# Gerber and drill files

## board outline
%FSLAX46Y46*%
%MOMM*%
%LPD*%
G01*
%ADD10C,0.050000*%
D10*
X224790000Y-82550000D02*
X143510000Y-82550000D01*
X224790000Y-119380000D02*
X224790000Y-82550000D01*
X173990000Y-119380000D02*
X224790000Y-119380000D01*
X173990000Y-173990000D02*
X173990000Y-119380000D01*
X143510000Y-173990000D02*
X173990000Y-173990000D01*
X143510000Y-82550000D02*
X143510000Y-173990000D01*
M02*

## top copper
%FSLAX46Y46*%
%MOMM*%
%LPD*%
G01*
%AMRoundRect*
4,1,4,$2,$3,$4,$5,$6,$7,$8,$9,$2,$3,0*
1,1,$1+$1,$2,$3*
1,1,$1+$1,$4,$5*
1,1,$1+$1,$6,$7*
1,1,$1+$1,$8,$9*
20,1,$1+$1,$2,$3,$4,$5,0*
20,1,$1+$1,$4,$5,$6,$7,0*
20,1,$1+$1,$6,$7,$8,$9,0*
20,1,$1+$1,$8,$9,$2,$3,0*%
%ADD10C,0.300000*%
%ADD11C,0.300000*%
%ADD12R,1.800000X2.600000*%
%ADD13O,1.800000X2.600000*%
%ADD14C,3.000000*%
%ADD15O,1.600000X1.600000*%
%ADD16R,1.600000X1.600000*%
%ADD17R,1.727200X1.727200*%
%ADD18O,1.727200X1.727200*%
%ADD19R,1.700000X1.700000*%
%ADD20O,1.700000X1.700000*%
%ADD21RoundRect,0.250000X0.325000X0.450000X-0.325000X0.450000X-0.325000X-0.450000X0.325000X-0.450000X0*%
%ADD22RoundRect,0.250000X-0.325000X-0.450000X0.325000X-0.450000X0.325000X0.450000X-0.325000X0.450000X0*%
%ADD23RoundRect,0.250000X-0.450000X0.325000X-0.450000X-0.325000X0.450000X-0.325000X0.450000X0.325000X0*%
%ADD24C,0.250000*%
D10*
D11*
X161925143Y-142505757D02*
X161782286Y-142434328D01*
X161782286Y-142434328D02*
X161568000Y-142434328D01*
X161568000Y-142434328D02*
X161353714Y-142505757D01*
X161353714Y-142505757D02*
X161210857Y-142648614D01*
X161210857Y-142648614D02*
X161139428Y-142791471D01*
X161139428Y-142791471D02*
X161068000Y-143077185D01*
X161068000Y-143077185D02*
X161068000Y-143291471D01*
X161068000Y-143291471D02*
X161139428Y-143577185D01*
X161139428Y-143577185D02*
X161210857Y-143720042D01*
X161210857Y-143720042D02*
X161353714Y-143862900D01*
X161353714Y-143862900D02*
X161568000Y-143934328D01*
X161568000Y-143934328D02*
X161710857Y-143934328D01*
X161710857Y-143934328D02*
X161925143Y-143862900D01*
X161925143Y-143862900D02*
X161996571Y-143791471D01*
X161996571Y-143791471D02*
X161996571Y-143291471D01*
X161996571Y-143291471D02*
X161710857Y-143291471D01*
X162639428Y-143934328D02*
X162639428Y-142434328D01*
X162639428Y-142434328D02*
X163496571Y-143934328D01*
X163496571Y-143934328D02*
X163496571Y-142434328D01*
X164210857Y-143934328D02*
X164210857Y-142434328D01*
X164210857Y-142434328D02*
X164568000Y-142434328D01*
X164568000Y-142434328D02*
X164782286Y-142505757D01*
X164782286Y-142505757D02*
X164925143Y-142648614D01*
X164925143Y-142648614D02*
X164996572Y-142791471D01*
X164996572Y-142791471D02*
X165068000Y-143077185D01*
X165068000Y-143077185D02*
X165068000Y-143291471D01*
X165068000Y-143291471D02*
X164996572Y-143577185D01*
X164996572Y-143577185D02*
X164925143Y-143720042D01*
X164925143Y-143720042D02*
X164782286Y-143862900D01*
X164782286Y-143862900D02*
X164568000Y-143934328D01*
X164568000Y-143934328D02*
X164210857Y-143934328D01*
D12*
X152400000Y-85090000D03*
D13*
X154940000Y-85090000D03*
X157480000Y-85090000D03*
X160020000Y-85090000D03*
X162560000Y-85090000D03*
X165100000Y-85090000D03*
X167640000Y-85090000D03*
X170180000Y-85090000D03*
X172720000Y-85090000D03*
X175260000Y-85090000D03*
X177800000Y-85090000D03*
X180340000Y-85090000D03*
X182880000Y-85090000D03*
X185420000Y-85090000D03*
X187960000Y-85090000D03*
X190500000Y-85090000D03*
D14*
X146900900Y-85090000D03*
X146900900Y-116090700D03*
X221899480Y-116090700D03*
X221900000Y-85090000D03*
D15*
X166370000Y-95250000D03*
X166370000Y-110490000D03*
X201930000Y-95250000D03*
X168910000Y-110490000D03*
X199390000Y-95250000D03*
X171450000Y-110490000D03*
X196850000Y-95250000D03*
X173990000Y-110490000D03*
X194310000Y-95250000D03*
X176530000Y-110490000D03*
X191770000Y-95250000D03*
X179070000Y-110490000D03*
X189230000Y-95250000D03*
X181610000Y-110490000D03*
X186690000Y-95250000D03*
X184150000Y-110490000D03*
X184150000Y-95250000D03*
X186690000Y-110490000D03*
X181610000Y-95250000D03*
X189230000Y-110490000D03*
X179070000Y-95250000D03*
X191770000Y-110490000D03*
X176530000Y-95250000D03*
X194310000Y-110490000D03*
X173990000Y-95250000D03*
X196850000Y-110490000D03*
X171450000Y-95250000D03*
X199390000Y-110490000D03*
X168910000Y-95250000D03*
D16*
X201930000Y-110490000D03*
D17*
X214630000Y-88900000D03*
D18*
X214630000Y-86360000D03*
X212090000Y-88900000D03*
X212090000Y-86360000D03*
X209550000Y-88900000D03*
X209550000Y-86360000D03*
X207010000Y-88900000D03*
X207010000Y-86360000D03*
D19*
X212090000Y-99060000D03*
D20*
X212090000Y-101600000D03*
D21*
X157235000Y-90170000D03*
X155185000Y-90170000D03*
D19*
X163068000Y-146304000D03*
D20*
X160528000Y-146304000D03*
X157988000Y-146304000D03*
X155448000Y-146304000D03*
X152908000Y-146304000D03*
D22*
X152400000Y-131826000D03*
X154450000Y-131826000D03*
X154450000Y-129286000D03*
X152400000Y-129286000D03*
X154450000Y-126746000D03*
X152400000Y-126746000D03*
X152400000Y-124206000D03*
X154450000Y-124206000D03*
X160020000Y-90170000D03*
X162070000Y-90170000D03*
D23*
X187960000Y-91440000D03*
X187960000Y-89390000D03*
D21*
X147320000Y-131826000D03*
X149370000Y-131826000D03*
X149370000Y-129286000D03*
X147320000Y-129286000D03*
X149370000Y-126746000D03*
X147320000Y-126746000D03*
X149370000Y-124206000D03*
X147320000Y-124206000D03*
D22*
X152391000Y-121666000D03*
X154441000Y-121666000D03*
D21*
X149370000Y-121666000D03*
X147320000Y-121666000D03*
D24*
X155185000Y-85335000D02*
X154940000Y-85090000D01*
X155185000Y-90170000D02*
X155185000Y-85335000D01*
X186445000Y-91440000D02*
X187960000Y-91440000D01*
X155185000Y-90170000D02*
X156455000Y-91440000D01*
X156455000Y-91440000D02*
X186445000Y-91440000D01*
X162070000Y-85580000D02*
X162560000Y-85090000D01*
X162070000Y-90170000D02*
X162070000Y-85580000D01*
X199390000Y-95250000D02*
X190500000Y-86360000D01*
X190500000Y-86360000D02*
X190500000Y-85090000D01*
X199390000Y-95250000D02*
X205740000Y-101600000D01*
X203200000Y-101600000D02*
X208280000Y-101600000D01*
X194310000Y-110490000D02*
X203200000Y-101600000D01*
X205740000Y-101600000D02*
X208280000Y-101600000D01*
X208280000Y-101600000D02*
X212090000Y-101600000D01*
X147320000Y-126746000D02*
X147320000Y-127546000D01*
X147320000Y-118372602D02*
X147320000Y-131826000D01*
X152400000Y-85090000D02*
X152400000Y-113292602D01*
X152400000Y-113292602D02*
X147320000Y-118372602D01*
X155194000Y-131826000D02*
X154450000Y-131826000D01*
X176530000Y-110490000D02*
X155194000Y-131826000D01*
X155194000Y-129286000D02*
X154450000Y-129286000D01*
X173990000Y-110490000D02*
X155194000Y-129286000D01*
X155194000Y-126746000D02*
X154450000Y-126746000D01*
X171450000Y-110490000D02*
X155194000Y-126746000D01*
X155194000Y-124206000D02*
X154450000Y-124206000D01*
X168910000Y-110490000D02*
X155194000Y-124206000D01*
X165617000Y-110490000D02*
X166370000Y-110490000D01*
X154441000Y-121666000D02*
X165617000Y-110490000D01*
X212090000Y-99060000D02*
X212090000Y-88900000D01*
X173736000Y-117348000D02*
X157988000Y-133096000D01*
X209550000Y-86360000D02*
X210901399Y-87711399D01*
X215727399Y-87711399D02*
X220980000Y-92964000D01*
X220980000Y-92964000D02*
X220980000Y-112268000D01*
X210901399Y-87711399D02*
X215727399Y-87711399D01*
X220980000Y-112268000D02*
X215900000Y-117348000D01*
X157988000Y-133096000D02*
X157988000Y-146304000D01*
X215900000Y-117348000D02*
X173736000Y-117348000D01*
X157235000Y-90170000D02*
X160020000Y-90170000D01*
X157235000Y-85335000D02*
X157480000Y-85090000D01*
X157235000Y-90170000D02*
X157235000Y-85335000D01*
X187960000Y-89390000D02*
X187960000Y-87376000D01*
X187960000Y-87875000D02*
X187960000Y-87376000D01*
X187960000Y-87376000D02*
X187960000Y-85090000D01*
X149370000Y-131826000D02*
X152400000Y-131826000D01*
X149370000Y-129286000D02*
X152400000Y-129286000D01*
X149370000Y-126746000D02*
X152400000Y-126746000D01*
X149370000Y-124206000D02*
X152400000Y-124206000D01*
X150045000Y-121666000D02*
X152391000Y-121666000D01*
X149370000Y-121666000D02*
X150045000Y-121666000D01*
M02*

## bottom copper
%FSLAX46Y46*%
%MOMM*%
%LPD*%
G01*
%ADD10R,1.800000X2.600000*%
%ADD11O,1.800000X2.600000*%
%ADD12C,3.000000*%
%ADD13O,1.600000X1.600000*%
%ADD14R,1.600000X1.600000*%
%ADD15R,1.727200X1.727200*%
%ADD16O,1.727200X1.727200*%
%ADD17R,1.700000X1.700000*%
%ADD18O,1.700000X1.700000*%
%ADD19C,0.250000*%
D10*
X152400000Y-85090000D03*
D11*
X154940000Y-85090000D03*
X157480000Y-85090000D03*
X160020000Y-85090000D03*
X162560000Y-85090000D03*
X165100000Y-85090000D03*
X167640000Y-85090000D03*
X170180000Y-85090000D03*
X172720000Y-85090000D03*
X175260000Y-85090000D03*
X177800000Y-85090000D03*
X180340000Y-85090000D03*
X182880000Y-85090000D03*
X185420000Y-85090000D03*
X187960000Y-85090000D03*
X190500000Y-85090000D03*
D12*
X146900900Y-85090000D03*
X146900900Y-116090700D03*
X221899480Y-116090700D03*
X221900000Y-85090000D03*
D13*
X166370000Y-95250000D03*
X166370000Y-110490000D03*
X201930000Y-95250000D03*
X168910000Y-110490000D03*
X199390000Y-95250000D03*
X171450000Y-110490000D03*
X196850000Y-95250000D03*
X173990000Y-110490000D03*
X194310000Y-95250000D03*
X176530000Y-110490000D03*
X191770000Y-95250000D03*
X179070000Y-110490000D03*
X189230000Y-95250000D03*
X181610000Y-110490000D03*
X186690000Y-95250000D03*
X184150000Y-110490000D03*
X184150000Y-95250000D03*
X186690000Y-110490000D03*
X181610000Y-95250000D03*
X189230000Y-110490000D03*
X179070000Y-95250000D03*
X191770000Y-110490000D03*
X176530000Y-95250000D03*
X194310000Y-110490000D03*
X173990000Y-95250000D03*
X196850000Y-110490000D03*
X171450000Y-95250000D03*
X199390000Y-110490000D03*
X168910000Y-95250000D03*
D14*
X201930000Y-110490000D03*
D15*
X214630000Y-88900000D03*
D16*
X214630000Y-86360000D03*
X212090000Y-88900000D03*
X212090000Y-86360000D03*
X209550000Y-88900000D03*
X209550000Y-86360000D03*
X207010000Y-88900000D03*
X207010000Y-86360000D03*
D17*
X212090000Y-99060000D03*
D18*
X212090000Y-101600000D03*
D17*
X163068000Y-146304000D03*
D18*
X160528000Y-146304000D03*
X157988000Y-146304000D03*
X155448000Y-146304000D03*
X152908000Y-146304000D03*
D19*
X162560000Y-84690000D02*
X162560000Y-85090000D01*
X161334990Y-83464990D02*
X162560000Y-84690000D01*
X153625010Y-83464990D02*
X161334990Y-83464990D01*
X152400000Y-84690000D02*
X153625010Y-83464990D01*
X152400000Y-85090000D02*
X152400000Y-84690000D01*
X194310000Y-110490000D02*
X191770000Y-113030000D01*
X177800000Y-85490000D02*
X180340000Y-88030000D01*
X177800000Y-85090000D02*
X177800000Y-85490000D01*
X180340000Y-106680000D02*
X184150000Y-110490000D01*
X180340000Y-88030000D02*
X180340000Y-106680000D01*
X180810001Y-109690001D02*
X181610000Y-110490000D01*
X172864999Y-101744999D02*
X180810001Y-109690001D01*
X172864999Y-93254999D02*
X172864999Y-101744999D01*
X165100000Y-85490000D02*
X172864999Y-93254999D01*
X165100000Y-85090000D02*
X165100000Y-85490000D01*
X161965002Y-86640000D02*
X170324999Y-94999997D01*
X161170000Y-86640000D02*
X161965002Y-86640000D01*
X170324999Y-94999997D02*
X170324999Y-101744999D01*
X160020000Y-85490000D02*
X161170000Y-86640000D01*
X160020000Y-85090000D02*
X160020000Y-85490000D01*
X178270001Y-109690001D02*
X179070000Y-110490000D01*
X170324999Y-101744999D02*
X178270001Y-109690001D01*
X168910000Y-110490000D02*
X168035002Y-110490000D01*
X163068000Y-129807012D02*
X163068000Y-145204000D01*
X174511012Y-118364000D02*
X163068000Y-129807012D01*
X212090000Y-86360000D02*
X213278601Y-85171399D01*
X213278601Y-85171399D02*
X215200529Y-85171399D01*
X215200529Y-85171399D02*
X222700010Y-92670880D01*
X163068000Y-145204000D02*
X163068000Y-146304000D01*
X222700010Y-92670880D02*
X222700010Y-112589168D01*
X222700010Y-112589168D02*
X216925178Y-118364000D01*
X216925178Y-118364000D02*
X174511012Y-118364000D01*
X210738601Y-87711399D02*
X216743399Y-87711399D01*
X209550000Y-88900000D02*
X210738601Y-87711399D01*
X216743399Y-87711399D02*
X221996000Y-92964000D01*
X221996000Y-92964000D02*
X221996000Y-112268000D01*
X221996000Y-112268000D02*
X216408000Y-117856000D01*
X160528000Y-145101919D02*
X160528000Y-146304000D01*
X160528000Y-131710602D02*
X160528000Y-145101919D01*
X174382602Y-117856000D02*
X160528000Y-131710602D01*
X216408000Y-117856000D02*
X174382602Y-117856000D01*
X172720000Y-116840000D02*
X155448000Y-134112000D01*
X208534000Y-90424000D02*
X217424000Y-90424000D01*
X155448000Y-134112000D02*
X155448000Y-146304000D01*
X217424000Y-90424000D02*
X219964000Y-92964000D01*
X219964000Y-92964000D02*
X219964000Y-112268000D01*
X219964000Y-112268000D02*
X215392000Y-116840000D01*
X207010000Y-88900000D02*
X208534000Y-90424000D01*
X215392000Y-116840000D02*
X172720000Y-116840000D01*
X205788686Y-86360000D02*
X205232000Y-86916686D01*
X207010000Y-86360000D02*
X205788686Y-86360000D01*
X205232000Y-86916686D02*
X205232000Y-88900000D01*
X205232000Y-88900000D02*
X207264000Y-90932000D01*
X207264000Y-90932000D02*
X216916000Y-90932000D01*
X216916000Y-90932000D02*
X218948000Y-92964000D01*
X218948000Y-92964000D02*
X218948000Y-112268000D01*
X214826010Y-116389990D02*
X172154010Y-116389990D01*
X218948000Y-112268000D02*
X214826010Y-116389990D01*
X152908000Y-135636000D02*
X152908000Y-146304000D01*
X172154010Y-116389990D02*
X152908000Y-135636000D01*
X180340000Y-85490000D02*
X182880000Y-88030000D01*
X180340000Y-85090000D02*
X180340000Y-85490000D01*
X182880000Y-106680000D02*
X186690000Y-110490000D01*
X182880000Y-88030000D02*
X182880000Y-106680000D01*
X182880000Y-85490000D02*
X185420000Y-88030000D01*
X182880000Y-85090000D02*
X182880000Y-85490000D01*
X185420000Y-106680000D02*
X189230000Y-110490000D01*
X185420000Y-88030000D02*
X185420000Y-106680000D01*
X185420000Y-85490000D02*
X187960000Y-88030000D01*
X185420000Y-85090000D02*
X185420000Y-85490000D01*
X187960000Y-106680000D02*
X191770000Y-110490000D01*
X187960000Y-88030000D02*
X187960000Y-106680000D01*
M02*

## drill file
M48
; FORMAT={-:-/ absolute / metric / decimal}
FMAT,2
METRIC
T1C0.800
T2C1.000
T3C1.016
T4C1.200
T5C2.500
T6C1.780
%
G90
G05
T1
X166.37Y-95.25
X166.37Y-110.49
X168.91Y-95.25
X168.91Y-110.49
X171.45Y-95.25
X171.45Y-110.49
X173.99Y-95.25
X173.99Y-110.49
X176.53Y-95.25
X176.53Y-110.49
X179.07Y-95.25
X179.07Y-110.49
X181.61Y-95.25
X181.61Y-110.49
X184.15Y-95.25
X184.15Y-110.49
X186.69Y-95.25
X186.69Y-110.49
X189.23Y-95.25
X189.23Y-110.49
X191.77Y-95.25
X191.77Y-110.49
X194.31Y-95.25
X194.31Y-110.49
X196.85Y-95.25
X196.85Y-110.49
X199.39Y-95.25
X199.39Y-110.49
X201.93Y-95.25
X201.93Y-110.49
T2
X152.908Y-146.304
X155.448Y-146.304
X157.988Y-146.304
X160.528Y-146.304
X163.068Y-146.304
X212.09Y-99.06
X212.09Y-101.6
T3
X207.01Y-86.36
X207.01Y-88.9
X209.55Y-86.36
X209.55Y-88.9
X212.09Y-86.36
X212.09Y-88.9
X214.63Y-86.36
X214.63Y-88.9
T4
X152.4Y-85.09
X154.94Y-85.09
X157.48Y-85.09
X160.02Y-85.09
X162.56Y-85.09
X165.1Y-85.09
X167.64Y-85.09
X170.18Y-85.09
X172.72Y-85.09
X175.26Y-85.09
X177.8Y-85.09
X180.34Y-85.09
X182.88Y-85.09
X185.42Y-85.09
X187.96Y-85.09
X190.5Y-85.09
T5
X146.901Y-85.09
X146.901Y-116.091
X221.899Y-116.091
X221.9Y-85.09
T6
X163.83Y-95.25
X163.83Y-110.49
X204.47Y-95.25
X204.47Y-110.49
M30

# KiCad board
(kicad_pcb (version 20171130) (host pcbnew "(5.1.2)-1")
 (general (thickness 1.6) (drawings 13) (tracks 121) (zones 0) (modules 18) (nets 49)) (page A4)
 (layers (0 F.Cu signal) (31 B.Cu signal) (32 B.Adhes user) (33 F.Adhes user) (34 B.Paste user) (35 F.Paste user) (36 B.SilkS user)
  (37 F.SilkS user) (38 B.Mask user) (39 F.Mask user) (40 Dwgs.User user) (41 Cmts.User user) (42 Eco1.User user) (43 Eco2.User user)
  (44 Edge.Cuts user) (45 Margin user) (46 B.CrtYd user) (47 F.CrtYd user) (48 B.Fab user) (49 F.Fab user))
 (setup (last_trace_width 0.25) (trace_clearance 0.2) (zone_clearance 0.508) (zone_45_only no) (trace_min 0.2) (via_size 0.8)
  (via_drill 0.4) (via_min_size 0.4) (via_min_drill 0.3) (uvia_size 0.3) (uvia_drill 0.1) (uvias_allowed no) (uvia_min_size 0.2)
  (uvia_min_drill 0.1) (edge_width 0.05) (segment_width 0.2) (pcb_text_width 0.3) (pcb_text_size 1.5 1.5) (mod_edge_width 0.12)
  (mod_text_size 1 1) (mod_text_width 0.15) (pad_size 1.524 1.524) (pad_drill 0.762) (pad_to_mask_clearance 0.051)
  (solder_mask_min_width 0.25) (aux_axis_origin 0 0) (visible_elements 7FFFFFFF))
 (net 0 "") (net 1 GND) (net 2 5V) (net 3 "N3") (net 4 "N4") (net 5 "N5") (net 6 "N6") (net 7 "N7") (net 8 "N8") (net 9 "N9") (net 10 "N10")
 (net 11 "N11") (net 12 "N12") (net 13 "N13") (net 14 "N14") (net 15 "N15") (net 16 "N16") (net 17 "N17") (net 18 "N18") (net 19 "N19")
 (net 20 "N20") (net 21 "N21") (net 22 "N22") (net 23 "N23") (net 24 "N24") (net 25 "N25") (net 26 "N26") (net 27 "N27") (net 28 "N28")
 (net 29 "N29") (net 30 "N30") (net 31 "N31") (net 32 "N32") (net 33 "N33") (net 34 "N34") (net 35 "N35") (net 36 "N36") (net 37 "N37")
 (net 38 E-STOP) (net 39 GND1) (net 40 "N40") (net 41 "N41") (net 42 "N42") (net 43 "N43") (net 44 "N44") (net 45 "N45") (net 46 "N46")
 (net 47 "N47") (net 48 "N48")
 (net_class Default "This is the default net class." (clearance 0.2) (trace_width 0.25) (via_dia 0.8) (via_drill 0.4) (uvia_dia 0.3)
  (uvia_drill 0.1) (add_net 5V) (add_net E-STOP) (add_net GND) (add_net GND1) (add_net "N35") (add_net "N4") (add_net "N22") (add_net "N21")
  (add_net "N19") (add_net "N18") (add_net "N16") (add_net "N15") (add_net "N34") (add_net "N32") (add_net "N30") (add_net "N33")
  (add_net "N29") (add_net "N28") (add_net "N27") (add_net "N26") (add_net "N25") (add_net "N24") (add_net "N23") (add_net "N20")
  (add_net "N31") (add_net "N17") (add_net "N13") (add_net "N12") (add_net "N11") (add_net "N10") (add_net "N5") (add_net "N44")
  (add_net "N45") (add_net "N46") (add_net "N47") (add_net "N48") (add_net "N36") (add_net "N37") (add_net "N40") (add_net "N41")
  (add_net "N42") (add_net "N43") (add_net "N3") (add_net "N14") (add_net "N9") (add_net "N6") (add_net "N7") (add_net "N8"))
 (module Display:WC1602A (layer F.Cu) (at 152.4 85.09)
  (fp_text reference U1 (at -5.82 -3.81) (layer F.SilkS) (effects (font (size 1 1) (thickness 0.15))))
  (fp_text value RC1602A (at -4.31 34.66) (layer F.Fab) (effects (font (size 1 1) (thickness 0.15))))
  (pad 1 thru_hole rect (at 0 0) (size 1.8 2.6) (drill 1.2) (layers *.Cu *.Mask) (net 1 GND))
  (pad 2 thru_hole oval (at 2.54 0) (size 1.8 2.6) (drill 1.2) (layers *.Cu *.Mask) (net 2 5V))
  (pad 3 thru_hole oval (at 5.08 0) (size 1.8 2.6) (drill 1.2) (layers *.Cu *.Mask) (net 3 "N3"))
  (pad 4 thru_hole oval (at 7.62 0) (size 1.8 2.6) (drill 1.2) (layers *.Cu *.Mask) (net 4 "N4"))
  (pad 5 thru_hole oval (at 10.16 0) (size 1.8 2.6) (drill 1.2) (layers *.Cu *.Mask) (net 1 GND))
  (pad 6 thru_hole oval (at 12.7 0) (size 1.8 2.6) (drill 1.2) (layers *.Cu *.Mask) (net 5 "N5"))
  (pad 7 thru_hole oval (at 15.24 0) (size 1.8 2.6) (drill 1.2) (layers *.Cu *.Mask) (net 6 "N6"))
  (pad 8 thru_hole oval (at 17.78 0) (size 1.8 2.6) (drill 1.2) (layers *.Cu *.Mask) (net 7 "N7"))
  (pad 9 thru_hole oval (at 20.32 0) (size 1.8 2.6) (drill 1.2) (layers *.Cu *.Mask) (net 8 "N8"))
  (pad 10 thru_hole oval (at 22.86 0) (size 1.8 2.6) (drill 1.2) (layers *.Cu *.Mask) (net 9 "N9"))
  (pad 11 thru_hole oval (at 25.4 0) (size 1.8 2.6) (drill 1.2) (layers *.Cu *.Mask) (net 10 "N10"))
  (pad 12 thru_hole oval (at 27.94 0) (size 1.8 2.6) (drill 1.2) (layers *.Cu *.Mask) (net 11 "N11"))
  (pad 13 thru_hole oval (at 30.48 0) (size 1.8 2.6) (drill 1.2) (layers *.Cu *.Mask) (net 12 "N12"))
  (pad 14 thru_hole oval (at 33.02 0) (size 1.8 2.6) (drill 1.2) (layers *.Cu *.Mask) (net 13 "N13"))
  (pad 15 thru_hole oval (at 35.56 0) (size 1.8 2.6) (drill 1.2) (layers *.Cu *.Mask) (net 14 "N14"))
  (pad 16 thru_hole oval (at 38.1 0) (size 1.8 2.6) (drill 1.2) (layers *.Cu *.Mask) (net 1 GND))
  (pad "" thru_hole circle (at -5.4991 0) (size 3 3) (drill 2.5) (layers *.Cu *.Mask))
  (pad "" thru_hole circle (at -5.4991 31.0007) (size 3 3) (drill 2.5) (layers *.Cu *.Mask))
  (pad "" thru_hole circle (at 69.49948 31.0007) (size 3 3) (drill 2.5) (layers *.Cu *.Mask))
  (pad "" thru_hole circle (at 69.5 0) (size 3 3) (drill 2.5) (layers *.Cu *.Mask)))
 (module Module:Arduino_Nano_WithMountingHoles (layer B.Cu) (at 201.93 110.49 90)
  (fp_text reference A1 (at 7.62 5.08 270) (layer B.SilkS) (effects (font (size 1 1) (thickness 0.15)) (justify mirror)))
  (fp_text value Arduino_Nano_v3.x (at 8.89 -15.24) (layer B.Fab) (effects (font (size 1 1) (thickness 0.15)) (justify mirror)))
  (pad "" np_thru_hole circle (at 0 -38.1 90) (size 1.78 1.78) (drill 1.78) (layers *.Cu *.Mask))
  (pad "" np_thru_hole circle (at 15.24 -38.1 90) (size 1.78 1.78) (drill 1.78) (layers *.Cu *.Mask))
  (pad "" np_thru_hole circle (at 15.24 2.54 90) (size 1.78 1.78) (drill 1.78) (layers *.Cu *.Mask))
  (pad "" np_thru_hole circle (at 0 2.54 90) (size 1.78 1.78) (drill 1.78) (layers *.Cu *.Mask))
  (pad 16 thru_hole oval (at 15.24 -35.56 90) (size 1.6 1.6) (drill 0.8) (layers *.Cu *.Mask) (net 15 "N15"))
  (pad 15 thru_hole oval (at 0 -35.56 90) (size 1.6 1.6) (drill 0.8) (layers *.Cu *.Mask) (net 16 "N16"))
  (pad 30 thru_hole oval (at 15.24 0 90) (size 1.6 1.6) (drill 0.8) (layers *.Cu *.Mask) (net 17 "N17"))
  (pad 14 thru_hole oval (at 0 -33.02 90) (size 1.6 1.6) (drill 0.8) (layers *.Cu *.Mask) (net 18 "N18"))
  (pad 29 thru_hole oval (at 15.24 -2.54 90) (size 1.6 1.6) (drill 0.8) (layers *.Cu *.Mask) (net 1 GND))
  (pad 13 thru_hole oval (at 0 -30.48 90) (size 1.6 1.6) (drill 0.8) (layers *.Cu *.Mask) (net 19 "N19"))
  (pad 28 thru_hole oval (at 15.24 -5.08 90) (size 1.6 1.6) (drill 0.8) (layers *.Cu *.Mask) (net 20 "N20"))
  (pad 12 thru_hole oval (at 0 -27.94 90) (size 1.6 1.6) (drill 0.8) (layers *.Cu *.Mask) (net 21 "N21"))
  (pad 27 thru_hole oval (at 15.24 -7.62 90) (size 1.6 1.6) (drill 0.8) (layers *.Cu *.Mask) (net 2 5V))
  (pad 11 thru_hole oval (at 0 -25.4 90) (size 1.6 1.6) (drill 0.8) (layers *.Cu *.Mask) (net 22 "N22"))
  (pad 26 thru_hole oval (at 15.24 -10.16 90) (size 1.6 1.6) (drill 0.8) (layers *.Cu *.Mask) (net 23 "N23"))
  (pad 10 thru_hole oval (at 0 -22.86 90) (size 1.6 1.6) (drill 0.8) (layers *.Cu *.Mask) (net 4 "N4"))
  (pad 25 thru_hole oval (at 15.24 -12.7 90) (size 1.6 1.6) (drill 0.8) (layers *.Cu *.Mask) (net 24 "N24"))
  (pad 9 thru_hole oval (at 0 -20.32 90) (size 1.6 1.6) (drill 0.8) (layers *.Cu *.Mask) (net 5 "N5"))
  (pad 24 thru_hole oval (at 15.24 -15.24 90) (size 1.6 1.6) (drill 0.8) (layers *.Cu *.Mask) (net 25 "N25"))
  (pad 8 thru_hole oval (at 0 -17.78 90) (size 1.6 1.6) (drill 0.8) (layers *.Cu *.Mask) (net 10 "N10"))
  (pad 23 thru_hole oval (at 15.24 -17.78 90) (size 1.6 1.6) (drill 0.8) (layers *.Cu *.Mask) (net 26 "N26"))
  (pad 7 thru_hole oval (at 0 -15.24 90) (size 1.6 1.6) (drill 0.8) (layers *.Cu *.Mask) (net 11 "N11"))
  (pad 22 thru_hole oval (at 15.24 -20.32 90) (size 1.6 1.6) (drill 0.8) (layers *.Cu *.Mask) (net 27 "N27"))
  (pad 6 thru_hole oval (at 0 -12.7 90) (size 1.6 1.6) (drill 0.8) (layers *.Cu *.Mask) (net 12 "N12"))
  (pad 21 thru_hole oval (at 15.24 -22.86 90) (size 1.6 1.6) (drill 0.8) (layers *.Cu *.Mask) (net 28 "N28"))
  (pad 5 thru_hole oval (at 0 -10.16 90) (size 1.6 1.6) (drill 0.8) (layers *.Cu *.Mask) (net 13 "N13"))
  (pad 20 thru_hole oval (at 15.24 -25.4 90) (size 1.6 1.6) (drill 0.8) (layers *.Cu *.Mask) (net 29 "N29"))
  (pad 4 thru_hole oval (at 0 -7.62 90) (size 1.6 1.6) (drill 0.8) (layers *.Cu *.Mask) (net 1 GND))
  (pad 19 thru_hole oval (at 15.24 -27.94 90) (size 1.6 1.6) (drill 0.8) (layers *.Cu *.Mask) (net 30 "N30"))
  (pad 3 thru_hole oval (at 0 -5.08 90) (size 1.6 1.6) (drill 0.8) (layers *.Cu *.Mask) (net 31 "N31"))
  (pad 18 thru_hole oval (at 15.24 -30.48 90) (size 1.6 1.6) (drill 0.8) (layers *.Cu *.Mask) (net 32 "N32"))
  (pad 2 thru_hole oval (at 0 -2.54 90) (size 1.6 1.6) (drill 0.8) (layers *.Cu *.Mask) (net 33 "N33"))
  (pad 17 thru_hole oval (at 15.24 -33.02 90) (size 1.6 1.6) (drill 0.8) (layers *.Cu *.Mask) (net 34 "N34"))
  (pad 1 thru_hole rect (at 0 0 90) (size 1.6 1.6) (drill 0.8) (layers *.Cu *.Mask) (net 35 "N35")))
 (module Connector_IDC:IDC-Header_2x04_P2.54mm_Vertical (layer B.Cu) (at 214.63 88.9 90)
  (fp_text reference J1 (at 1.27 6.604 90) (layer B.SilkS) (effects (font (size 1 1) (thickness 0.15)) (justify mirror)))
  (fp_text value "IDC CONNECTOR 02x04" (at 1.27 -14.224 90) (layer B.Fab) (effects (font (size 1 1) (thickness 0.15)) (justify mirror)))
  (pad 1 thru_hole rect (at 0 0 90) (size 1.7272 1.7272) (drill 1.016) (layers *.Cu *.Mask) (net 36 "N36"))
  (pad 2 thru_hole oval (at 2.54 0 90) (size 1.7272 1.7272) (drill 1.016) (layers *.Cu *.Mask) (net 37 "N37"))
  (pad 3 thru_hole oval (at 0 -2.54 90) (size 1.7272 1.7272) (drill 1.016) (layers *.Cu *.Mask) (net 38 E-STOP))
  (pad 4 thru_hole oval (at 2.54 -2.54 90) (size 1.7272 1.7272) (drill 1.016) (layers *.Cu *.Mask) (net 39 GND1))
  (pad 5 thru_hole oval (at 0 -5.08 90) (size 1.7272 1.7272) (drill 1.016) (layers *.Cu *.Mask) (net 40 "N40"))
  (pad 6 thru_hole oval (at 2.54 -5.08 90) (size 1.7272 1.7272) (drill 1.016) (layers *.Cu *.Mask) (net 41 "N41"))
  (pad 7 thru_hole oval (at 0 -7.62 90) (size 1.7272 1.7272) (drill 1.016) (layers *.Cu *.Mask) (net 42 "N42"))
  (pad 8 thru_hole oval (at 2.54 -7.62 90) (size 1.7272 1.7272) (drill 1.016) (layers *.Cu *.Mask) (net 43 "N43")))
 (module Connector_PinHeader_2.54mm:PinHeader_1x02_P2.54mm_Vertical (layer B.Cu) (at 212.09 99.06 180)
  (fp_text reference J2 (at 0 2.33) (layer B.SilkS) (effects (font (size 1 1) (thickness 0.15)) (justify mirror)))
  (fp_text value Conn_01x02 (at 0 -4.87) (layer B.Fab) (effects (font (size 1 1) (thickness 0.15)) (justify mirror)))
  (pad 1 thru_hole rect (at 0 0 180) (size 1.7 1.7) (drill 1) (layers *.Cu *.Mask) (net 38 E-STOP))
  (pad 2 thru_hole oval (at 0 -2.54 180) (size 1.7 1.7) (drill 1) (layers *.Cu *.Mask) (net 1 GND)))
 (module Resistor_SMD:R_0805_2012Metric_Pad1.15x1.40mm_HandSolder (layer F.Cu) (at 156.21 90.17 180)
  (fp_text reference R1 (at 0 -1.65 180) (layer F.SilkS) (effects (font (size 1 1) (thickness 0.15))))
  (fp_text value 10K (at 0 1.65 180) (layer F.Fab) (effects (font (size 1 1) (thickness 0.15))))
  (pad 1 smd roundrect (at -1.025 0 180) (size 1.15 1.4) (layers F.Cu F.Paste F.Mask) (roundrect_rratio 0.217391) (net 3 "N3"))
  (pad 2 smd roundrect (at 1.025 0 180) (size 1.15 1.4) (layers F.Cu F.Paste F.Mask) (roundrect_rratio 0.217391) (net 2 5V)))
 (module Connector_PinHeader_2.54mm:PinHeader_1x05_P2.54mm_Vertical (layer F.Cu) (at 163.068 146.304 270)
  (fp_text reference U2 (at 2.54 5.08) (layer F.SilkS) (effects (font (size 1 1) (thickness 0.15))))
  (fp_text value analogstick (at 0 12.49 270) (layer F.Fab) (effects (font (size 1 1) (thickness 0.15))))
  (pad 1 thru_hole rect (at 0 0 270) (size 1.7 1.7) (drill 1) (layers *.Cu *.Mask) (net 39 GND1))
  (pad 2 thru_hole oval (at 0 2.54 270) (size 1.7 1.7) (drill 1) (layers *.Cu *.Mask) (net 40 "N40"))
  (pad 3 thru_hole oval (at 0 5.08 270) (size 1.7 1.7) (drill 1) (layers *.Cu *.Mask) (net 41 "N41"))
  (pad 4 thru_hole oval (at 0 7.62 270) (size 1.7 1.7) (drill 1) (layers *.Cu *.Mask) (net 42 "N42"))
  (pad 5 thru_hole oval (at 0 10.16 270) (size 1.7 1.7) (drill 1) (layers *.Cu *.Mask) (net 43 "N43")))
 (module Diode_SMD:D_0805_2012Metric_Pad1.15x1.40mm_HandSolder (layer F.Cu) (at 153.425 131.826)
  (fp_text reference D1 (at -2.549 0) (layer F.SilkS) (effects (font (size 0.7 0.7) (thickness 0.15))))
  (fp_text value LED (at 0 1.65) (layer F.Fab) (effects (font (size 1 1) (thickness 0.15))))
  (pad 1 smd roundrect (at -1.025 0) (size 1.15 1.4) (layers F.Cu F.Paste F.Mask) (roundrect_rratio 0.217391) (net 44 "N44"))
  (pad 2 smd roundrect (at 1.025 0) (size 1.15 1.4) (layers F.Cu F.Paste F.Mask) (roundrect_rratio 0.217391) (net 22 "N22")))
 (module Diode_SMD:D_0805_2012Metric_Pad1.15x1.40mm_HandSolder (layer F.Cu) (at 153.425 129.286)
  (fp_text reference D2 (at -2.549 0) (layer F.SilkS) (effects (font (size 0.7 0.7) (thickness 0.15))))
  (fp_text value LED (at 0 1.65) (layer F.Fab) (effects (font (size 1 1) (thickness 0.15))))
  (pad 2 smd roundrect (at 1.025 0) (size 1.15 1.4) (layers F.Cu F.Paste F.Mask) (roundrect_rratio 0.217391) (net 21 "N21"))
  (pad 1 smd roundrect (at -1.025 0) (size 1.15 1.4) (layers F.Cu F.Paste F.Mask) (roundrect_rratio 0.217391) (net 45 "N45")))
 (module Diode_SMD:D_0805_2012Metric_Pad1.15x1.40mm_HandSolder (layer F.Cu) (at 153.425 126.746)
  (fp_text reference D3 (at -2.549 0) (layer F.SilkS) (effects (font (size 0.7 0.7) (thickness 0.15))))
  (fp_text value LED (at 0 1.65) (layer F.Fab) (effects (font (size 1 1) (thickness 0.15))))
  (pad 2 smd roundrect (at 1.025 0) (size 1.15 1.4) (layers F.Cu F.Paste F.Mask) (roundrect_rratio 0.217391) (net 19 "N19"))
  (pad 1 smd roundrect (at -1.025 0) (size 1.15 1.4) (layers F.Cu F.Paste F.Mask) (roundrect_rratio 0.217391) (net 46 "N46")))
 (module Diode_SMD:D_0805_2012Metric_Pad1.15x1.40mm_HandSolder (layer F.Cu) (at 153.425 124.206)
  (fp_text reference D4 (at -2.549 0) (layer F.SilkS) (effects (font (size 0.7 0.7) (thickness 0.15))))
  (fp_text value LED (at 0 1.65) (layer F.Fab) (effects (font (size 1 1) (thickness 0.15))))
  (pad 1 smd roundrect (at -1.025 0) (size 1.15 1.4) (layers F.Cu F.Paste F.Mask) (roundrect_rratio 0.217391) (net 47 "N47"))
  (pad 2 smd roundrect (at 1.025 0) (size 1.15 1.4) (layers F.Cu F.Paste F.Mask) (roundrect_rratio 0.217391) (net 18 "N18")))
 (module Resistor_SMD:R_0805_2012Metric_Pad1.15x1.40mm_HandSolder (layer F.Cu) (at 161.045 90.17)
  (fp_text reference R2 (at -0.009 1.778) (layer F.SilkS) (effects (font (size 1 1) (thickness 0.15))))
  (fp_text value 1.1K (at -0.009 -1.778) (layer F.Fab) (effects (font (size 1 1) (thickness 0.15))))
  (pad 1 smd roundrect (at -1.025 0) (size 1.15 1.4) (layers F.Cu F.Paste F.Mask) (roundrect_rratio 0.217391) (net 3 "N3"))
  (pad 2 smd roundrect (at 1.025 0) (size 1.15 1.4) (layers F.Cu F.Paste F.Mask) (roundrect_rratio 0.217391) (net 1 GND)))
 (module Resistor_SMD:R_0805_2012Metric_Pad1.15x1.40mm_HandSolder (layer F.Cu) (at 187.96 90.415 270)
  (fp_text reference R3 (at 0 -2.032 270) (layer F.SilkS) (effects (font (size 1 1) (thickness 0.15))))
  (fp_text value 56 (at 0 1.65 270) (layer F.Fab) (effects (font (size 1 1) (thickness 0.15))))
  (pad 2 smd roundrect (at 1.025 0 270) (size 1.15 1.4) (layers F.Cu F.Paste F.Mask) (roundrect_rratio 0.217391) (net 2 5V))
  (pad 1 smd roundrect (at -1.025 0 270) (size 1.15 1.4) (layers F.Cu F.Paste F.Mask) (roundrect_rratio 0.217391) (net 14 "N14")))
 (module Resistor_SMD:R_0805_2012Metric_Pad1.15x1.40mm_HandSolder (layer F.Cu) (at 148.345 131.826 180)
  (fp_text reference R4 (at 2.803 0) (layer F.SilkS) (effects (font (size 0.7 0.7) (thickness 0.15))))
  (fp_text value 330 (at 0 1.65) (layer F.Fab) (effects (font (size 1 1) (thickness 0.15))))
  (pad 2 smd roundrect (at 1.025 0 180) (size 1.15 1.4) (layers F.Cu F.Paste F.Mask) (roundrect_rratio 0.217391) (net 1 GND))
  (pad 1 smd roundrect (at -1.025 0 180) (size 1.15 1.4) (layers F.Cu F.Paste F.Mask) (roundrect_rratio 0.217391) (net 44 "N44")))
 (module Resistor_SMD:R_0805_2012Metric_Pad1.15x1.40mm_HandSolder (layer F.Cu) (at 148.345 129.286 180)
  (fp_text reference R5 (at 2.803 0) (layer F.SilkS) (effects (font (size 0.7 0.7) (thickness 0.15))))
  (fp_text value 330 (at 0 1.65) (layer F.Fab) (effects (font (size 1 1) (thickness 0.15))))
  (pad 1 smd roundrect (at -1.025 0 180) (size 1.15 1.4) (layers F.Cu F.Paste F.Mask) (roundrect_rratio 0.217391) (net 45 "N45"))
  (pad 2 smd roundrect (at 1.025 0 180) (size 1.15 1.4) (layers F.Cu F.Paste F.Mask) (roundrect_rratio 0.217391) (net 1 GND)))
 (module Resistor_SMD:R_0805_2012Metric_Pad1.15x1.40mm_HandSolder (layer F.Cu) (at 148.345 126.746 180)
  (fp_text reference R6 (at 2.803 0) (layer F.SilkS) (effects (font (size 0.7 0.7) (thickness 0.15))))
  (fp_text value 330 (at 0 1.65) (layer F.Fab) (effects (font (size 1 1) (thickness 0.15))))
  (pad 1 smd roundrect (at -1.025 0 180) (size 1.15 1.4) (layers F.Cu F.Paste F.Mask) (roundrect_rratio 0.217391) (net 46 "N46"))
  (pad 2 smd roundrect (at 1.025 0 180) (size 1.15 1.4) (layers F.Cu F.Paste F.Mask) (roundrect_rratio 0.217391) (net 1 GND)))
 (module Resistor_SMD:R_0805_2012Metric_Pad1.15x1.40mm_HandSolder (layer F.Cu) (at 148.345 124.206 180)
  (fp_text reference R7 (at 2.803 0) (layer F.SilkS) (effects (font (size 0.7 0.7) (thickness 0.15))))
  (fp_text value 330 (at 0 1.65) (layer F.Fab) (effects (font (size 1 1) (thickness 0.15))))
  (pad 1 smd roundrect (at -1.025 0 180) (size 1.15 1.4) (layers F.Cu F.Paste F.Mask) (roundrect_rratio 0.217391) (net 47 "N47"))
  (pad 2 smd roundrect (at 1.025 0 180) (size 1.15 1.4) (layers F.Cu F.Paste F.Mask) (roundrect_rratio 0.217391) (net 1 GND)))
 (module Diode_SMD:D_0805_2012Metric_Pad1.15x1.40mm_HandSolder (layer F.Cu) (at 153.416 121.666)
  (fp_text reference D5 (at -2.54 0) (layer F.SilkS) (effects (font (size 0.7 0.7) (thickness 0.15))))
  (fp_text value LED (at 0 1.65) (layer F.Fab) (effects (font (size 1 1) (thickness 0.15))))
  (pad 1 smd roundrect (at -1.025 0) (size 1.15 1.4) (layers F.Cu F.Paste F.Mask) (roundrect_rratio 0.217391) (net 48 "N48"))
  (pad 2 smd roundrect (at 1.025 0) (size 1.15 1.4) (layers F.Cu F.Paste F.Mask) (roundrect_rratio 0.217391) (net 16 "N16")))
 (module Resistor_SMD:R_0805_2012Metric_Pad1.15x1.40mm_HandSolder (layer F.Cu) (at 148.345 121.666 180)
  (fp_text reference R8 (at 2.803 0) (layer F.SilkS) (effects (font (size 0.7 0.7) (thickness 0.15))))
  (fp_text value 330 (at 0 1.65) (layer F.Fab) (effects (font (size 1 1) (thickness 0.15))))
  (pad 1 smd roundrect (at -1.025 0 180) (size 1.15 1.4) (layers F.Cu F.Paste F.Mask) (roundrect_rratio 0.217391) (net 48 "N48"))
  (pad 2 smd roundrect (at 1.025 0 180) (size 1.15 1.4) (layers F.Cu F.Paste F.Mask) (roundrect_rratio 0.217391) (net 1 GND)))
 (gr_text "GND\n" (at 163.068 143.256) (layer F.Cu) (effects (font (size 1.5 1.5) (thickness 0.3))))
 (gr_line (start 224.79 82.55) (end 143.51 82.55) (layer Edge.Cuts) (width 0.05))
 (gr_line (start 224.79 119.38) (end 224.79 82.55) (layer Edge.Cuts) (width 0.05))
 (gr_line (start 173.99 119.38) (end 224.79 119.38) (layer Edge.Cuts) (width 0.05))
 (gr_line (start 173.99 173.99) (end 173.99 119.38) (layer Edge.Cuts) (width 0.05))
 (gr_line (start 143.51 173.99) (end 173.99 173.99) (layer Edge.Cuts) (width 0.05))
 (gr_line (start 143.51 82.55) (end 143.51 173.99) (layer Edge.Cuts) (width 0.05))
 (segment (start 155.185 85.335) (end 154.94 85.09) (width 0.25) (layer F.Cu) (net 2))
 (segment (start 155.185 90.17) (end 155.185 85.335) (width 0.25) (layer F.Cu) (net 2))
 (segment (start 186.445 91.44) (end 187.96 91.44) (width 0.25) (layer F.Cu) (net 2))
 (segment (start 155.185 90.17) (end 156.455 91.44) (width 0.25) (layer F.Cu) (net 2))
 (segment (start 156.455 91.44) (end 186.445 91.44) (width 0.25) (layer F.Cu) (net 2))
 (segment (start 162.07 85.58) (end 162.56 85.09) (width 0.25) (layer F.Cu) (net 1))
 (segment (start 162.07 90.17) (end 162.07 85.58) (width 0.25) (layer F.Cu) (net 1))
 (segment (start 199.39 95.25) (end 190.5 86.36) (width 0.25) (layer F.Cu) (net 1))
 (segment (start 190.5 86.36) (end 190.5 85.09) (width 0.25) (layer F.Cu) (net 1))
 (segment (start 199.39 95.25) (end 205.74 101.6) (width 0.25) (layer F.Cu) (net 1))
 (segment (start 203.2 101.6) (end 208.28 101.6) (width 0.25) (layer F.Cu) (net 1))
 (segment (start 194.31 110.49) (end 203.2 101.6) (width 0.25) (layer F.Cu) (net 1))
 (segment (start 205.74 101.6) (end 208.28 101.6) (width 0.25) (layer F.Cu) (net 1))
 (segment (start 208.28 101.6) (end 212.09 101.6) (width 0.25) (layer F.Cu) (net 1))
 (segment (start 162.56 84.69) (end 162.56 85.09) (width 0.25) (layer B.Cu) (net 1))
 (segment (start 161.33499 83.46499) (end 162.56 84.69) (width 0.25) (layer B.Cu) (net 1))
 (segment (start 153.62501 83.46499) (end 161.33499 83.46499) (width 0.25) (layer B.Cu) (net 1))
 (segment (start 152.4 84.69) (end 153.62501 83.46499) (width 0.25) (layer B.Cu) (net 1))
 (segment (start 152.4 85.09) (end 152.4 84.69) (width 0.25) (layer B.Cu) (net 1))
 (segment (start 194.31 110.49) (end 191.77 113.03) (width 0.25) (layer B.Cu) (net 1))
 (segment (start 147.32 126.746) (end 147.32 127.546) (width 0.25) (layer F.Cu) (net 1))
 (segment (start 147.32 118.372602) (end 147.32 131.826) (width 0.25) (layer F.Cu) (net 1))
 (segment (start 152.4 85.09) (end 152.4 113.292602) (width 0.25) (layer F.Cu) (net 1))
 (segment (start 152.4 113.292602) (end 147.32 118.372602) (width 0.25) (layer F.Cu) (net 1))
 (segment (start 177.8 85.49) (end 180.34 88.03) (width 0.25) (layer B.Cu) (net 10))
 (segment (start 177.8 85.09) (end 177.8 85.49) (width 0.25) (layer B.Cu) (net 10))
 (segment (start 180.34 106.68) (end 184.15 110.49) (width 0.25) (layer B.Cu) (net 10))
 (segment (start 180.34 88.03) (end 180.34 106.68) (width 0.25) (layer B.Cu) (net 10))
 (segment (start 180.810001 109.690001) (end 181.61 110.49) (width 0.25) (layer B.Cu) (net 5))
 (segment (start 172.864999 101.744999) (end 180.810001 109.690001) (width 0.25) (layer B.Cu) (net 5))
 (segment (start 172.864999 93.254999) (end 172.864999 101.744999) (width 0.25) (layer B.Cu) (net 5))
 (segment (start 165.1 85.49) (end 172.864999 93.254999) (width 0.25) (layer B.Cu) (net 5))
 (segment (start 165.1 85.09) (end 165.1 85.49) (width 0.25) (layer B.Cu) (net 5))
 (segment (start 161.965002 86.64) (end 170.324999 94.999997) (width 0.25) (layer B.Cu) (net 4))
 (segment (start 161.17 86.64) (end 161.965002 86.64) (width 0.25) (layer B.Cu) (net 4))
 (segment (start 170.324999 94.999997) (end 170.324999 101.744999) (width 0.25) (layer B.Cu) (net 4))
 (segment (start 160.02 85.49) (end 161.17 86.64) (width 0.25) (layer B.Cu) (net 4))
 (segment (start 160.02 85.09) (end 160.02 85.49) (width 0.25) (layer B.Cu) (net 4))
 (segment (start 178.270001 109.690001) (end 179.07 110.49) (width 0.25) (layer B.Cu) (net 4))
 (segment (start 170.324999 101.744999) (end 178.270001 109.690001) (width 0.25) (layer B.Cu) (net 4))
 (segment (start 155.194 131.826) (end 154.45 131.826) (width 0.25) (layer F.Cu) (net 22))
 (segment (start 176.53 110.49) (end 155.194 131.826) (width 0.25) (layer F.Cu) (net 22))
 (segment (start 155.194 129.286) (end 154.45 129.286) (width 0.25) (layer F.Cu) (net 21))
 (segment (start 173.99 110.49) (end 155.194 129.286) (width 0.25) (layer F.Cu) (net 21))
 (segment (start 155.194 126.746) (end 154.45 126.746) (width 0.25) (layer F.Cu) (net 19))
 (segment (start 171.45 110.49) (end 155.194 126.746) (width 0.25) (layer F.Cu) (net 19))
 (segment (start 168.91 110.49) (end 168.035002 110.49) (width 0.25) (layer B.Cu) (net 18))
 (segment (start 155.194 124.206) (end 154.45 124.206) (width 0.25) (layer F.Cu) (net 18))
 (segment (start 168.91 110.49) (end 155.194 124.206) (width 0.25) (layer F.Cu) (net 18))
 (segment (start 165.617 110.49) (end 166.37 110.49) (width 0.25) (layer F.Cu) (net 16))
 (segment (start 154.441 121.666) (end 165.617 110.49) (width 0.25) (layer F.Cu) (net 16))
 (segment (start 212.09 99.06) (end 212.09 88.9) (width 0.25) (layer F.Cu) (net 38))
 (segment (start 163.068 129.807012) (end 163.068 145.204) (width 0.25) (layer B.Cu) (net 39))
 (segment (start 174.511012 118.364) (end 163.068 129.807012) (width 0.25) (layer B.Cu) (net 39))
 (segment (start 212.09 86.36) (end 213.278601 85.171399) (width 0.25) (layer B.Cu) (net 39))
 (segment (start 213.278601 85.171399) (end 215.200529 85.171399) (width 0.25) (layer B.Cu) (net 39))
 (segment (start 215.200529 85.171399) (end 222.70001 92.67088) (width 0.25) (layer B.Cu) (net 39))
 (segment (start 163.068 145.204) (end 163.068 146.304) (width 0.25) (layer B.Cu) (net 39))
 (segment (start 222.70001 92.67088) (end 222.70001 112.589168) (width 0.25) (layer B.Cu) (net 39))
 (segment (start 222.70001 112.589168) (end 216.925178 118.364) (width 0.25) (layer B.Cu) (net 39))
 (segment (start 216.925178 118.364) (end 174.511012 118.364) (width 0.25) (layer B.Cu) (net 39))
 (segment (start 210.738601 87.711399) (end 216.743399 87.711399) (width 0.25) (layer B.Cu) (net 40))
 (segment (start 209.55 88.9) (end 210.738601 87.711399) (width 0.25) (layer B.Cu) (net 40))
 (segment (start 216.743399 87.711399) (end 221.996 92.964) (width 0.25) (layer B.Cu) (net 40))
 (segment (start 221.996 92.964) (end 221.996 112.268) (width 0.25) (layer B.Cu) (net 40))
 (segment (start 221.996 112.268) (end 216.408 117.856) (width 0.25) (layer B.Cu) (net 40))
 (segment (start 160.528 145.101919) (end 160.528 146.304) (width 0.25) (layer B.Cu) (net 40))
 (segment (start 160.528 131.710602) (end 160.528 145.101919) (width 0.25) (layer B.Cu) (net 40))
 (segment (start 174.382602 117.856) (end 160.528 131.710602) (width 0.25) (layer B.Cu) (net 40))
 (segment (start 216.408 117.856) (end 174.382602 117.856) (width 0.25) (layer B.Cu) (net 40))
 (segment (start 173.736 117.348) (end 157.988 133.096) (width 0.25) (layer F.Cu) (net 41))
 (segment (start 209.55 86.36) (end 210.901399 87.711399) (width 0.25) (layer F.Cu) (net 41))
 (segment (start 215.727399 87.711399) (end 220.98 92.964) (width 0.25) (layer F.Cu) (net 41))
 (segment (start 220.98 92.964) (end 220.98 112.268) (width 0.25) (layer F.Cu) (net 41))
 (segment (start 210.901399 87.711399) (end 215.727399 87.711399) (width 0.25) (layer F.Cu) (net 41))
 (segment (start 220.98 112.268) (end 215.9 117.348) (width 0.25) (layer F.Cu) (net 41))
 (segment (start 157.988 133.096) (end 157.988 146.304) (width 0.25) (layer F.Cu) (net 41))
 (segment (start 215.9 117.348) (end 173.736 117.348) (width 0.25) (layer F.Cu) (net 41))
 (segment (start 172.72 116.84) (end 155.448 134.112) (width 0.25) (layer B.Cu) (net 42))
 (segment (start 208.534 90.424) (end 217.424 90.424) (width 0.25) (layer B.Cu) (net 42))
 (segment (start 155.448 134.112) (end 155.448 146.304) (width 0.25) (layer B.Cu) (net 42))
 (segment (start 217.424 90.424) (end 219.964 92.964) (width 0.25) (layer B.Cu) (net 42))
 (segment (start 219.964 92.964) (end 219.964 112.268) (width 0.25) (layer B.Cu) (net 42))
 (segment (start 219.964 112.268) (end 215.392 116.84) (width 0.25) (layer B.Cu) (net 42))
 (segment (start 207.01 88.9) (end 208.534 90.424) (width 0.25) (layer B.Cu) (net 42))
 (segment (start 215.392 116.84) (end 172.72 116.84) (width 0.25) (layer B.Cu) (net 42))
 (segment (start 205.788686 86.36) (end 205.232 86.916686) (width 0.25) (layer B.Cu) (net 43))
 (segment (start 207.01 86.36) (end 205.788686 86.36) (width 0.25) (layer B.Cu) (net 43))
 (segment (start 205.232 86.916686) (end 205.232 88.9) (width 0.25) (layer B.Cu) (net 43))
 (segment (start 205.232 88.9) (end 207.264 90.932) (width 0.25) (layer B.Cu) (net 43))
 (segment (start 207.264 90.932) (end 216.916 90.932) (width 0.25) (layer B.Cu) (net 43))
 (segment (start 216.916 90.932) (end 218.948 92.964) (width 0.25) (layer B.Cu) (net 43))
 (segment (start 218.948 92.964) (end 218.948 112.268) (width 0.25) (layer B.Cu) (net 43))
 (segment (start 214.82601 116.38999) (end 172.15401 116.38999) (width 0.25) (layer B.Cu) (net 43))
 (segment (start 218.948 112.268) (end 214.82601 116.38999) (width 0.25) (layer B.Cu) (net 43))
 (segment (start 152.908 135.636) (end 152.908 146.304) (width 0.25) (layer B.Cu) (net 43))
 (segment (start 172.15401 116.38999) (end 152.908 135.636) (width 0.25) (layer B.Cu) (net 43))
 (segment (start 157.235 90.17) (end 160.02 90.17) (width 0.25) (layer F.Cu) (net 3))
 (segment (start 157.235 85.335) (end 157.48 85.09) (width 0.25) (layer F.Cu) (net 3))
 (segment (start 157.235 90.17) (end 157.235 85.335) (width 0.25) (layer F.Cu) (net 3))
 (segment (start 187.96 89.39) (end 187.96 87.376) (width 0.25) (layer F.Cu) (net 14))
 (segment (start 187.96 87.875) (end 187.96 87.376) (width 0.25) (layer F.Cu) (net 14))
 (segment (start 187.96 87.376) (end 187.96 85.09) (width 0.25) (layer F.Cu) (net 14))
 (segment (start 180.34 85.49) (end 182.88 88.03) (width 0.25) (layer B.Cu) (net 11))
 (segment (start 180.34 85.09) (end 180.34 85.49) (width 0.25) (layer B.Cu) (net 11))
 (segment (start 182.88 106.68) (end 186.69 110.49) (width 0.25) (layer B.Cu) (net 11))
 (segment (start 182.88 88.03) (end 182.88 106.68) (width 0.25) (layer B.Cu) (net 11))
 (segment (start 182.88 85.49) (end 185.42 88.03) (width 0.25) (layer B.Cu) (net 12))
 (segment (start 182.88 85.09) (end 182.88 85.49) (width 0.25) (layer B.Cu) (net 12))
 (segment (start 185.42 106.68) (end 189.23 110.49) (width 0.25) (layer B.Cu) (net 12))
 (segment (start 185.42 88.03) (end 185.42 106.68) (width 0.25) (layer B.Cu) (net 12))
 (segment (start 185.42 85.49) (end 187.96 88.03) (width 0.25) (layer B.Cu) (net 13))
 (segment (start 185.42 85.09) (end 185.42 85.49) (width 0.25) (layer B.Cu) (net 13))
 (segment (start 187.96 106.68) (end 191.77 110.49) (width 0.25) (layer B.Cu) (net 13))
 (segment (start 187.96 88.03) (end 187.96 106.68) (width 0.25) (layer B.Cu) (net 13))
 (segment (start 149.37 131.826) (end 152.4 131.826) (width 0.25) (layer F.Cu) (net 44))
 (segment (start 149.37 129.286) (end 152.4 129.286) (width 0.25) (layer F.Cu) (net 45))
 (segment (start 149.37 126.746) (end 152.4 126.746) (width 0.25) (layer F.Cu) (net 46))
 (segment (start 149.37 124.206) (end 152.4 124.206) (width 0.25) (layer F.Cu) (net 47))
 (segment (start 150.045 121.666) (end 152.391 121.666) (width 0.25) (layer F.Cu) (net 48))
 (segment (start 149.37 121.666) (end 150.045 121.666) (width 0.25) (layer F.Cu) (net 48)))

